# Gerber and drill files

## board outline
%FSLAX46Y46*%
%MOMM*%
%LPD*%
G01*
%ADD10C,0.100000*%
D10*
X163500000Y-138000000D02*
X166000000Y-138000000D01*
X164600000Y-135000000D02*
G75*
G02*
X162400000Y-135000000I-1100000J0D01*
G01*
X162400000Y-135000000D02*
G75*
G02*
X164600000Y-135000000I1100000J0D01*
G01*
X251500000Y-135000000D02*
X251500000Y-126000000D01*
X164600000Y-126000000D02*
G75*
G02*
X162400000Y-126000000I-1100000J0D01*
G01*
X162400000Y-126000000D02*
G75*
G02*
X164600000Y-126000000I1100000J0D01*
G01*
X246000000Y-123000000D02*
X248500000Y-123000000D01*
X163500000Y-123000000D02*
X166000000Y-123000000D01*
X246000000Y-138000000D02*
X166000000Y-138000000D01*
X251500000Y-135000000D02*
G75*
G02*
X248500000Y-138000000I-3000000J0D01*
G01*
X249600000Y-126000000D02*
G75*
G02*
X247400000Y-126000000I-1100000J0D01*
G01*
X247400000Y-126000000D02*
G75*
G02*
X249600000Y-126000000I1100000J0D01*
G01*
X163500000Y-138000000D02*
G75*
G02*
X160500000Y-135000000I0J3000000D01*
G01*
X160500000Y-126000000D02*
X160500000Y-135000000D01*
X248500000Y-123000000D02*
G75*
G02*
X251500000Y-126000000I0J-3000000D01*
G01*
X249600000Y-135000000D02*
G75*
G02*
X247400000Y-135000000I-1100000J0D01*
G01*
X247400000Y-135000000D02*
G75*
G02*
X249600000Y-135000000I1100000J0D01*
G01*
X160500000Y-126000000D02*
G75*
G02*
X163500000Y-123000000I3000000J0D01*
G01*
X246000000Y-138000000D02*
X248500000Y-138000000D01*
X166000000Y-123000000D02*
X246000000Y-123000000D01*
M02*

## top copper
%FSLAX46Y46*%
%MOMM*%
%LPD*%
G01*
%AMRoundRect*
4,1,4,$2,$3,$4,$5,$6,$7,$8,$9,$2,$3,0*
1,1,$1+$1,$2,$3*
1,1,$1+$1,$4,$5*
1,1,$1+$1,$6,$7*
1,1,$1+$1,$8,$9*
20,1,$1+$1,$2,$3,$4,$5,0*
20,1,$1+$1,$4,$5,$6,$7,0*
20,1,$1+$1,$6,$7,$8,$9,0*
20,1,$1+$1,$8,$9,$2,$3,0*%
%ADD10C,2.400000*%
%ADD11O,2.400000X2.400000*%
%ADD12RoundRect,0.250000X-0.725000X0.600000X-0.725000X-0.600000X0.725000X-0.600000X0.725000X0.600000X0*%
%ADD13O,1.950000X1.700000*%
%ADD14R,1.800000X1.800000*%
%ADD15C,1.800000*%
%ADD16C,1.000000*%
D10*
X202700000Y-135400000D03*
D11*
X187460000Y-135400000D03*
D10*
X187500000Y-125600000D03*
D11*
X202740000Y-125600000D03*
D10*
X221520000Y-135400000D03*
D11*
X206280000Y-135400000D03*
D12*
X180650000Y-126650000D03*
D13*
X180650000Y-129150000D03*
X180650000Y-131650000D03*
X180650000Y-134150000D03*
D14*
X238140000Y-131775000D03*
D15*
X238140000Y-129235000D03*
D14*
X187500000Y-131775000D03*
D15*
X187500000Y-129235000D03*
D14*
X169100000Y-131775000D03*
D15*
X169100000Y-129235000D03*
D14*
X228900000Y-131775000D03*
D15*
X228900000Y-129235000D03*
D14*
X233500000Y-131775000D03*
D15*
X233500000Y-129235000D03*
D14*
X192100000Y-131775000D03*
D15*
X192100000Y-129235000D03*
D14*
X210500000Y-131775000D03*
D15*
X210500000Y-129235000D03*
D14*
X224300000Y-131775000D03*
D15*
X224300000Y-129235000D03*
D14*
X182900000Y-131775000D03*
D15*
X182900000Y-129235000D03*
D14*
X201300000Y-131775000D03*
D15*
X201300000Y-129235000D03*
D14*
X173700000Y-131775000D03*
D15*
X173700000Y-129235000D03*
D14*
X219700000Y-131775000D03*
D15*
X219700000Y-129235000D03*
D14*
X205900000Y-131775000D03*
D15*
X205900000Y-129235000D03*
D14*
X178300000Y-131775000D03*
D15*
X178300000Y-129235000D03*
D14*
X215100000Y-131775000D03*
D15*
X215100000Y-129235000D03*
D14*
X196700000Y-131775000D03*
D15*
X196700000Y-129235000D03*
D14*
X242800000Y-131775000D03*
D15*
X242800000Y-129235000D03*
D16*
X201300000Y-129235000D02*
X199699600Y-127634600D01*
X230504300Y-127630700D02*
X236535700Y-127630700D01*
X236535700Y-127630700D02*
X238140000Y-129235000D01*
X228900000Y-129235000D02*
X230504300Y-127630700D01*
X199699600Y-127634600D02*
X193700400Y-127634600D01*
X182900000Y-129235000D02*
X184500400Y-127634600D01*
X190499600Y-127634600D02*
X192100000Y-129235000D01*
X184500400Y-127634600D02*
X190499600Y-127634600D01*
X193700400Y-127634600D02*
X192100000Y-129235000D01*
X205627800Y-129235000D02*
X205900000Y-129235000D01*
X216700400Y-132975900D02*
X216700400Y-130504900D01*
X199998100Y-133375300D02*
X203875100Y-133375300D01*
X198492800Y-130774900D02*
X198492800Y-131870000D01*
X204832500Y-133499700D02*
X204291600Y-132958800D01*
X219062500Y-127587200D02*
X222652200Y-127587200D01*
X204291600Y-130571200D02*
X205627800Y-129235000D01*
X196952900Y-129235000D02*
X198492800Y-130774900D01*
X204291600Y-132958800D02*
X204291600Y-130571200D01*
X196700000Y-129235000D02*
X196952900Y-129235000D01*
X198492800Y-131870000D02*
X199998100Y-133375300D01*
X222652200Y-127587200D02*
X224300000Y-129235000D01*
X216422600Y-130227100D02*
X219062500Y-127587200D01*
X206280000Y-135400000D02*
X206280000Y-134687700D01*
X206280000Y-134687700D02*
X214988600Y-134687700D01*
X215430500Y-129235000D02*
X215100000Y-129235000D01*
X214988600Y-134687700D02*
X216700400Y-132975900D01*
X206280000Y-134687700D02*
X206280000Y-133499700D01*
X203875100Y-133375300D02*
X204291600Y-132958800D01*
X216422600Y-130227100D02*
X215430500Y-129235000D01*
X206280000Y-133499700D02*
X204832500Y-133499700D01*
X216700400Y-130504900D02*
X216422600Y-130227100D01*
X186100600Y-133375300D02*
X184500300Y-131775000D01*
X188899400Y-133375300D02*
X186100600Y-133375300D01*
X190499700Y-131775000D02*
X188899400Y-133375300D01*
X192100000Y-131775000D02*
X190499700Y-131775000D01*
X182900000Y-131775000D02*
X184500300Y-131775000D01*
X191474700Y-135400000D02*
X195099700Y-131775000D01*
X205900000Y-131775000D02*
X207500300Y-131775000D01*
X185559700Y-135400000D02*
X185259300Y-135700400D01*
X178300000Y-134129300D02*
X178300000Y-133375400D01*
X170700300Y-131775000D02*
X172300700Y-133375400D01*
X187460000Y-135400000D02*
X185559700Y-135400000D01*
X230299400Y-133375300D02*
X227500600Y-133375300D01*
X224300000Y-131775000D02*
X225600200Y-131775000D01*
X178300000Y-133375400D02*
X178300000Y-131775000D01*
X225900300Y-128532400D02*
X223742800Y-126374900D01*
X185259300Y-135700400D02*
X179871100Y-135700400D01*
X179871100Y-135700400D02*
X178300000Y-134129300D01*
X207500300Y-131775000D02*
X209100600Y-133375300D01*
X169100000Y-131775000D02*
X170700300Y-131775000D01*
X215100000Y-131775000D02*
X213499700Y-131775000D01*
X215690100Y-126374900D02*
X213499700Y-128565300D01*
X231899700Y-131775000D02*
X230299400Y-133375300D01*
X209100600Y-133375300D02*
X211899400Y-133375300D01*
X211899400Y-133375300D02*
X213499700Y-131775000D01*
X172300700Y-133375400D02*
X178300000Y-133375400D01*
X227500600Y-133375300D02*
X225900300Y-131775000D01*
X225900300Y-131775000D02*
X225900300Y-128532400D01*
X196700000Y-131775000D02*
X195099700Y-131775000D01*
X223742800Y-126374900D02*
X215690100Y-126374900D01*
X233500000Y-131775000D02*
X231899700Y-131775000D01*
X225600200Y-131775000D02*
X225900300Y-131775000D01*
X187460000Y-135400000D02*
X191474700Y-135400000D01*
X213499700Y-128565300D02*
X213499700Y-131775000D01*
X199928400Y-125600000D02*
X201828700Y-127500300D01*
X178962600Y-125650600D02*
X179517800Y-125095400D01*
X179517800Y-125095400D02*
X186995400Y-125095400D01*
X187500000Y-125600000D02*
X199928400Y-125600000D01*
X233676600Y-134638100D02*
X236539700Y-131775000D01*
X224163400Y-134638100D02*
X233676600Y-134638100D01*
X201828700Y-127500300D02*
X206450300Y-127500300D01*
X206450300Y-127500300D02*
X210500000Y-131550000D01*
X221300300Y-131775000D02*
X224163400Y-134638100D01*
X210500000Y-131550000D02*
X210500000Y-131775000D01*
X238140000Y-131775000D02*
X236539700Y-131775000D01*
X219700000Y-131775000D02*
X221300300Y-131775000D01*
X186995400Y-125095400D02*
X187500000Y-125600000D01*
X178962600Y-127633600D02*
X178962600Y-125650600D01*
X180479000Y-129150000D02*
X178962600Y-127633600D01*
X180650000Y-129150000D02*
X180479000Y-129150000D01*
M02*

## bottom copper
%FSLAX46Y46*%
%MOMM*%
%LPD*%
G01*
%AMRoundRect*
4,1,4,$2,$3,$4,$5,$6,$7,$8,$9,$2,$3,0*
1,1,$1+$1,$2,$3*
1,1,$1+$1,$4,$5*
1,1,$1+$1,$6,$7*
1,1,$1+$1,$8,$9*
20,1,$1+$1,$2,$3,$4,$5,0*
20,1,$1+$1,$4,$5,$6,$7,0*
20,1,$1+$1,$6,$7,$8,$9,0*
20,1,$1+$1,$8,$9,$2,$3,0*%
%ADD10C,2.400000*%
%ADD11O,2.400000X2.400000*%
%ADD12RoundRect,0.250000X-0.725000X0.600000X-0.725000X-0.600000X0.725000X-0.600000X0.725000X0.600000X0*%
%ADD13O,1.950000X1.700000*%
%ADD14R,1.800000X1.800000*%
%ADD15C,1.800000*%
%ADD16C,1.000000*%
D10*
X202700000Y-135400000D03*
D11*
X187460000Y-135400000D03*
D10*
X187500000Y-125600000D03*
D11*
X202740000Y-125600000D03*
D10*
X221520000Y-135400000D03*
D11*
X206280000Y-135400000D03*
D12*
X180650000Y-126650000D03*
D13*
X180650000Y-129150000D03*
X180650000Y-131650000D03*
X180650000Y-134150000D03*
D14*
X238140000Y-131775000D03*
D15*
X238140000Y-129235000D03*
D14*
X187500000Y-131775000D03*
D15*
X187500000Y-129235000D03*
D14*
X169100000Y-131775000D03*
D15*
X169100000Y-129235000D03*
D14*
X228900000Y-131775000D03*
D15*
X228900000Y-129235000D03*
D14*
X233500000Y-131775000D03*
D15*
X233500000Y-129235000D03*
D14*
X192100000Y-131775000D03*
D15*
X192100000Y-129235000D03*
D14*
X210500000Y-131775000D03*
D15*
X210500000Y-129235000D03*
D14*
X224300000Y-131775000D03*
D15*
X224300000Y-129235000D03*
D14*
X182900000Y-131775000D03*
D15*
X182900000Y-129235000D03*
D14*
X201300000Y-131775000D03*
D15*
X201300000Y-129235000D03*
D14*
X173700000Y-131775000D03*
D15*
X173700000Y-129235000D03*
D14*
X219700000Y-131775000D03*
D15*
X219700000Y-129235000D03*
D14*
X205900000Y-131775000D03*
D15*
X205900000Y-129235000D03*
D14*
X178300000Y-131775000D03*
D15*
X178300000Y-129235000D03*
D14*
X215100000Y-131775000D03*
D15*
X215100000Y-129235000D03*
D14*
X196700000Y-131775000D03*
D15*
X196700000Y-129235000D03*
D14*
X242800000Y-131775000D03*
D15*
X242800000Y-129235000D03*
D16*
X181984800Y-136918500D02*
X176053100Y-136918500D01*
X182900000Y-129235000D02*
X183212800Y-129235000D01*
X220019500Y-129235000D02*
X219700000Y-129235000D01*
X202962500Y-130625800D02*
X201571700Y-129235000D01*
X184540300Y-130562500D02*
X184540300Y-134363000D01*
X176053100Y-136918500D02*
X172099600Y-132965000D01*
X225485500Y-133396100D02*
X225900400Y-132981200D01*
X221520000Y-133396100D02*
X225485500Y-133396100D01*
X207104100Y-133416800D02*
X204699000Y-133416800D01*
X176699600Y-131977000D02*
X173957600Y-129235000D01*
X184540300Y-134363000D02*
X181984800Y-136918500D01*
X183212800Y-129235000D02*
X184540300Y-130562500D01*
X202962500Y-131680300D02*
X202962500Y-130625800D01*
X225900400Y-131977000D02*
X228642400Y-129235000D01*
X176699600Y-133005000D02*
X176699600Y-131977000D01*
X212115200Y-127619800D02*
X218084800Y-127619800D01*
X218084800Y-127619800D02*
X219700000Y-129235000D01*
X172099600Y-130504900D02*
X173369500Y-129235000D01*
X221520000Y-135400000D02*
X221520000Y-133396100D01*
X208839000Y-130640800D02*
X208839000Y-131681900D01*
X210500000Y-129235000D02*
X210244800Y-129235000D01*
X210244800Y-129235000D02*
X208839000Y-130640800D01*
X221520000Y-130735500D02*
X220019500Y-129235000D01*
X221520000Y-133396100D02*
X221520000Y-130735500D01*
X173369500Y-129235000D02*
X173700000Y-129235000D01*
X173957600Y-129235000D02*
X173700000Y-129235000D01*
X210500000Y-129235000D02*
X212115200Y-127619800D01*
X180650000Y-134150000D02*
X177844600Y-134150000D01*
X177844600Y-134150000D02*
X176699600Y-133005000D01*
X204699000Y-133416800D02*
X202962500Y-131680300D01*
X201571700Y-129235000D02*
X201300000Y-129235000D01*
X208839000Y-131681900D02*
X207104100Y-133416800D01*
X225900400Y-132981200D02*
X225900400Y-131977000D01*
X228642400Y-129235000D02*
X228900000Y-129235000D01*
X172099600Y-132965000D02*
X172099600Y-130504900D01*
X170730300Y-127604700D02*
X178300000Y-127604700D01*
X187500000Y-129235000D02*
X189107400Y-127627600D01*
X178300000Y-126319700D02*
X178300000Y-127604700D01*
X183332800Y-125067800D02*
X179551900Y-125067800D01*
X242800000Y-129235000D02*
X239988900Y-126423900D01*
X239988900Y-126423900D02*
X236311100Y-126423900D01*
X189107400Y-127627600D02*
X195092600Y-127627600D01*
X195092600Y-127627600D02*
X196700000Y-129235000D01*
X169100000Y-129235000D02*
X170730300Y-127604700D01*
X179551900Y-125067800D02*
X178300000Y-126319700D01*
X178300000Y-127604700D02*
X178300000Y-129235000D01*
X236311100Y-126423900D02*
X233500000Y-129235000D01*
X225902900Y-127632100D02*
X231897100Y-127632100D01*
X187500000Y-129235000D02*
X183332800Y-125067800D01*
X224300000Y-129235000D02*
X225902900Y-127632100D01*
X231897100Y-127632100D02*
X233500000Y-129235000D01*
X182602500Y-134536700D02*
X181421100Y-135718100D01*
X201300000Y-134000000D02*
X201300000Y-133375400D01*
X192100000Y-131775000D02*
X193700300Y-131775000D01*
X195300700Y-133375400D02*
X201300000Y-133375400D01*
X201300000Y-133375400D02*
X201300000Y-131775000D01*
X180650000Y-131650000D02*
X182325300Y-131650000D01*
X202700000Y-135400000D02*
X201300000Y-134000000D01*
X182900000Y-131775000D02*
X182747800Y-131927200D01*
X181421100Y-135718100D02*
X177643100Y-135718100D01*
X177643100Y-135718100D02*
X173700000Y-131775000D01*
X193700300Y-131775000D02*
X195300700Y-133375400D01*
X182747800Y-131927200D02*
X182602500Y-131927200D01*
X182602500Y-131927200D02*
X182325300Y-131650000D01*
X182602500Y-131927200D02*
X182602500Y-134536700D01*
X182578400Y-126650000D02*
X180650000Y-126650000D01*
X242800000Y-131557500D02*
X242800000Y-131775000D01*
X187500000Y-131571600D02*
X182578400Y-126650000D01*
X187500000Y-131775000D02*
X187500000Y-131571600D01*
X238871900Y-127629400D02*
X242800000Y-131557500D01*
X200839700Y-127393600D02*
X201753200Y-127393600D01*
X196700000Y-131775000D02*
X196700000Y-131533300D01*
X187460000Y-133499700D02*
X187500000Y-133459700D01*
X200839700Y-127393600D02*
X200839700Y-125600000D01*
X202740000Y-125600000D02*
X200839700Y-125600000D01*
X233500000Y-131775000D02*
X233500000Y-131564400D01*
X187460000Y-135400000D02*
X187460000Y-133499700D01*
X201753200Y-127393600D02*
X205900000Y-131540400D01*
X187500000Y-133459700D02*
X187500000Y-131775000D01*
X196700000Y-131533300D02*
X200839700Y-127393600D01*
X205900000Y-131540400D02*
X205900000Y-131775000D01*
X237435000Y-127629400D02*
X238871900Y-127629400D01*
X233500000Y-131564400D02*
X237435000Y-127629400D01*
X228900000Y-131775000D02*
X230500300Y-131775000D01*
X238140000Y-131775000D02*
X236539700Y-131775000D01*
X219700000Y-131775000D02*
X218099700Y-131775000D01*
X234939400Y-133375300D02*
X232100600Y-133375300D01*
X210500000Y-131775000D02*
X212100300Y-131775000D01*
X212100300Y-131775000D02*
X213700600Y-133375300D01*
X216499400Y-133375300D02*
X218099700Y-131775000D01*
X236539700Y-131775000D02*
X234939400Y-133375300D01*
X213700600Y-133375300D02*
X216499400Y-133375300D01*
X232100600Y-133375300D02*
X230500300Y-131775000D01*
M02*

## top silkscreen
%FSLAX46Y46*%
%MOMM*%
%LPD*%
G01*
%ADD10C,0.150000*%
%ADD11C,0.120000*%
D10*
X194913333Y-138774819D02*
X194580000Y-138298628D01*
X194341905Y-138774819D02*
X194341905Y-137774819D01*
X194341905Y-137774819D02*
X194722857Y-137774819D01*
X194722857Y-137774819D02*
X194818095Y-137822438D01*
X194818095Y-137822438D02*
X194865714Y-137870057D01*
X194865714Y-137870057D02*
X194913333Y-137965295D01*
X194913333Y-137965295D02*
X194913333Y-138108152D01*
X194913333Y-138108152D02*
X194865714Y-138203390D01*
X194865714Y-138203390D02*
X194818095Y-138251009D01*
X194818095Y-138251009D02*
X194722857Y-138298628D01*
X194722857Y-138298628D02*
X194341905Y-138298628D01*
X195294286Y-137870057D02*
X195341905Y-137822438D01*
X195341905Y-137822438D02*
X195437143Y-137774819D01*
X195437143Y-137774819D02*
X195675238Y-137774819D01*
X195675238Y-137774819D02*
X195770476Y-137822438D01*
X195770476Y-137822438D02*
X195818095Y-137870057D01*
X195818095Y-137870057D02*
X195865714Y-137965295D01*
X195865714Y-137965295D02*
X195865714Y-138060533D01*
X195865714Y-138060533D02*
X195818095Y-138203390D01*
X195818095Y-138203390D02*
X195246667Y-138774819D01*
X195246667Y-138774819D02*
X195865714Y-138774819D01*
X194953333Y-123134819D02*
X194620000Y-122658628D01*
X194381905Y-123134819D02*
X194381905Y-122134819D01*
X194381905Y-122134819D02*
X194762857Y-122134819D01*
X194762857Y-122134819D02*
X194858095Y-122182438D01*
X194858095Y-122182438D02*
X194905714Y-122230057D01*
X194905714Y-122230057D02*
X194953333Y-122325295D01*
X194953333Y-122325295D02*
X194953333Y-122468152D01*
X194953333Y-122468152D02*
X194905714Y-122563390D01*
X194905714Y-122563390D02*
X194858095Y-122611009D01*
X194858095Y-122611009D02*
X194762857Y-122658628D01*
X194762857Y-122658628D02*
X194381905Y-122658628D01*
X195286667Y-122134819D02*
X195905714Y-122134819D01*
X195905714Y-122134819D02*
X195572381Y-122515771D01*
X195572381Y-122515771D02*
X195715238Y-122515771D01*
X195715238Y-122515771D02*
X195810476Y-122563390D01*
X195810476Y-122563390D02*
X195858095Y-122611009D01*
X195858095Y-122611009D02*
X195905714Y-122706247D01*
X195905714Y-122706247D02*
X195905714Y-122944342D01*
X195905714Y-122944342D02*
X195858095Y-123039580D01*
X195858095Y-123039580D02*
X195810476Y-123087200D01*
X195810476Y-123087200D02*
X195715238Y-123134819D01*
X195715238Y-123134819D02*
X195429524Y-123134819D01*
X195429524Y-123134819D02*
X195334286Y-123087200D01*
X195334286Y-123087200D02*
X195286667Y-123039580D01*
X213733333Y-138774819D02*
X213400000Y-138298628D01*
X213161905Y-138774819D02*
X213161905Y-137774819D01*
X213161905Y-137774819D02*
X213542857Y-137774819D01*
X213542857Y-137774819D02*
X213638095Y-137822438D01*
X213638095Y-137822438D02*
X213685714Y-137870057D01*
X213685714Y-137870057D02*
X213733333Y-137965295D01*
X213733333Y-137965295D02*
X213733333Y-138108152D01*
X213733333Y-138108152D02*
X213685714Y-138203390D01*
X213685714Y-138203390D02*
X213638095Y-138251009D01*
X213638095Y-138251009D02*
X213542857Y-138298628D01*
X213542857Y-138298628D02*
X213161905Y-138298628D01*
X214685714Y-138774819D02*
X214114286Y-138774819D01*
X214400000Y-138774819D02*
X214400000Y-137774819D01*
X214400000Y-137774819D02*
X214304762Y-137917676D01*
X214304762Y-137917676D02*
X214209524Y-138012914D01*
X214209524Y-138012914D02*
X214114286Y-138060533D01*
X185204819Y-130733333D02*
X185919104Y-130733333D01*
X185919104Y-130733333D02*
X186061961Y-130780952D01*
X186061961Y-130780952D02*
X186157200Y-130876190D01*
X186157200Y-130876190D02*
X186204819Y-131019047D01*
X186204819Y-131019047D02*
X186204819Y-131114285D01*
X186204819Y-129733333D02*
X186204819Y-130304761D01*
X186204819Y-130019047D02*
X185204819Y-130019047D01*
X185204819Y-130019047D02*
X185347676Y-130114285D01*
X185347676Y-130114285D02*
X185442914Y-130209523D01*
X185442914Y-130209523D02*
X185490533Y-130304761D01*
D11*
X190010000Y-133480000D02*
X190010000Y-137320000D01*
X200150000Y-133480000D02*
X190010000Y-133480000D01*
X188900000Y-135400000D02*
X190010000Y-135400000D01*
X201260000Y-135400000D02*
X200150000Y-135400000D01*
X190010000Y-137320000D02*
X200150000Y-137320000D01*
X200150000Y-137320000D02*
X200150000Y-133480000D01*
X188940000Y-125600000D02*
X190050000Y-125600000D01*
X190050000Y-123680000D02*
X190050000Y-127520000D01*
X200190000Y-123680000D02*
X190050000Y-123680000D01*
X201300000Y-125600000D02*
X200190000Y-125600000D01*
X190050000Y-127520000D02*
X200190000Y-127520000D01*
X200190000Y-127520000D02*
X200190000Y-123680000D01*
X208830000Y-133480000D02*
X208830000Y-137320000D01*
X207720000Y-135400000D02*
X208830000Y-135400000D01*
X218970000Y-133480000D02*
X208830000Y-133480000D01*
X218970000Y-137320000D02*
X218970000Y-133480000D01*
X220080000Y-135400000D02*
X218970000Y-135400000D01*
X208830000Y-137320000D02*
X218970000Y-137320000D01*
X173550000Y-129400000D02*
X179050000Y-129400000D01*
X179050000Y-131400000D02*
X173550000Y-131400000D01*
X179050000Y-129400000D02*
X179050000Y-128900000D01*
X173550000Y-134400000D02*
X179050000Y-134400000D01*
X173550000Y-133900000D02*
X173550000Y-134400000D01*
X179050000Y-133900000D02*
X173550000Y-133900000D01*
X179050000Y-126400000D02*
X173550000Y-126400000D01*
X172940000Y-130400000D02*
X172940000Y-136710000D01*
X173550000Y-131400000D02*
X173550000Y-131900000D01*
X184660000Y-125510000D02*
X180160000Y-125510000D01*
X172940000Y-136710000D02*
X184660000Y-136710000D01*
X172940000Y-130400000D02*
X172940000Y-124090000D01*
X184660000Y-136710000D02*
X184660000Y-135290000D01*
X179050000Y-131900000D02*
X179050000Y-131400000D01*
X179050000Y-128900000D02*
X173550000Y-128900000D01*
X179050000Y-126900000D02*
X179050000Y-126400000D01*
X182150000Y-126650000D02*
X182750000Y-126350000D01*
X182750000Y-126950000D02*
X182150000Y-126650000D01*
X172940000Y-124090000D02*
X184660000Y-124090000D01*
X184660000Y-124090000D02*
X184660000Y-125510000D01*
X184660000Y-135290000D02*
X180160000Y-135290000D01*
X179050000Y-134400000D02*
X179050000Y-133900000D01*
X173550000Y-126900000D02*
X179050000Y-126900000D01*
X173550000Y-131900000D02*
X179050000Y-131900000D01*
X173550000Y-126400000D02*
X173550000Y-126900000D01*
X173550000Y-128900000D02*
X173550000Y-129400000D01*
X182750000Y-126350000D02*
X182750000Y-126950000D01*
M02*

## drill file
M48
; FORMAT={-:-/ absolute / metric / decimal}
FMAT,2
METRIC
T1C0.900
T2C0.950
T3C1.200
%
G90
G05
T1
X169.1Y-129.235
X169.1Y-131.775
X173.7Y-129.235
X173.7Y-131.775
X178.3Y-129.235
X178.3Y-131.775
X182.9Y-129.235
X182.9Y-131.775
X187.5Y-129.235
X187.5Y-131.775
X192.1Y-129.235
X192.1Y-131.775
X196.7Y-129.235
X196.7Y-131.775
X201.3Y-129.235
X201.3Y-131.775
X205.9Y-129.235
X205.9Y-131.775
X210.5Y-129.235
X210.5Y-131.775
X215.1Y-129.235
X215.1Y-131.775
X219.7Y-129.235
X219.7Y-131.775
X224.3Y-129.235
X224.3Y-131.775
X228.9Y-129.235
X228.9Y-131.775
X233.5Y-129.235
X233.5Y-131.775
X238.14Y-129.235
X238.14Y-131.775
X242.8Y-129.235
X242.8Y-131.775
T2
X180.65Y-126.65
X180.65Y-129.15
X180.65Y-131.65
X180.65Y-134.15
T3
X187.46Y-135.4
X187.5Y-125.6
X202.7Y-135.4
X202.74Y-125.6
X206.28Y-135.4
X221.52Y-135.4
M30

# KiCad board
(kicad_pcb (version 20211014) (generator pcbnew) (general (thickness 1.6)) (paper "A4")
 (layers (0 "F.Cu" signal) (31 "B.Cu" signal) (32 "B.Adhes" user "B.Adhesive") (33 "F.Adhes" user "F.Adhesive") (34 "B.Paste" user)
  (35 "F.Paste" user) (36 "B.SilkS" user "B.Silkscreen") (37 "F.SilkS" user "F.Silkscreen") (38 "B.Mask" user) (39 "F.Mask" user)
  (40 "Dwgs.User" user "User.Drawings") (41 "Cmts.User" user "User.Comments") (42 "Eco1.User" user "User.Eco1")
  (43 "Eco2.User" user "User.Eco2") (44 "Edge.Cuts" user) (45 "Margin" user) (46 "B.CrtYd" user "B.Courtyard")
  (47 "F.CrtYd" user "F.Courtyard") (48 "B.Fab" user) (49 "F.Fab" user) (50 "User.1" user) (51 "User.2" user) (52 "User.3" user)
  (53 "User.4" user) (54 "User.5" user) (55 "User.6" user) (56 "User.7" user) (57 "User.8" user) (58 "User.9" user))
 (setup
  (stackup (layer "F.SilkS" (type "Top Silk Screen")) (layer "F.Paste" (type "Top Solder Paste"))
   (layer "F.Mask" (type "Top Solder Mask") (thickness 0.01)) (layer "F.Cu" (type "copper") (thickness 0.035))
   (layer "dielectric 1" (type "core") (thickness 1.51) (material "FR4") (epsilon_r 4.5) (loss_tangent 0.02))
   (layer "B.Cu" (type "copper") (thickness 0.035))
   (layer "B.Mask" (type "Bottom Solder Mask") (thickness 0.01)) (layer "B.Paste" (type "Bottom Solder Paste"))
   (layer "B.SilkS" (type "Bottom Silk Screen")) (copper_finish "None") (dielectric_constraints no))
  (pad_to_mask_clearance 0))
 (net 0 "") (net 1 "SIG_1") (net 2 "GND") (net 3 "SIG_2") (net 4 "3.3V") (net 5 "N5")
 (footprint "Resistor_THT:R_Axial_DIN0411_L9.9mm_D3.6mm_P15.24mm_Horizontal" (layer "F.Cu") (at 202.7 135.4 180)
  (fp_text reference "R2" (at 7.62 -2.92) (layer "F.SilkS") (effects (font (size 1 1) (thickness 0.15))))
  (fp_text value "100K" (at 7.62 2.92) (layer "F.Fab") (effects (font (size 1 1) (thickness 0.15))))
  (fp_line (start 12.69 1.92) (end 12.69 -1.92) (layer "F.SilkS") (width 0.12))
  (fp_line (start 2.55 1.92) (end 12.69 1.92) (layer "F.SilkS") (width 0.12))
  (fp_line (start 13.8 0) (end 12.69 0) (layer "F.SilkS") (width 0.12))
  (fp_line (start 1.44 0) (end 2.55 0) (layer "F.SilkS") (width 0.12))
  (fp_line (start 12.69 -1.92) (end 2.55 -1.92) (layer "F.SilkS") (width 0.12))
  (fp_line (start 2.55 -1.92) (end 2.55 1.92) (layer "F.SilkS") (width 0.12))
  (pad "1" thru_hole circle (at 0 0 180) (size 2.4 2.4) (drill 1.2) (layers *.Cu *.Mask) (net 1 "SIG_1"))
  (pad "2" thru_hole oval (at 15.24 0 180) (size 2.4 2.4) (drill 1.2) (layers *.Cu *.Mask) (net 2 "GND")))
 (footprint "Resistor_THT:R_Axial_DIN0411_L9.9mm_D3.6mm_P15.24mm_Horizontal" (layer "F.Cu") (at 187.5 125.6)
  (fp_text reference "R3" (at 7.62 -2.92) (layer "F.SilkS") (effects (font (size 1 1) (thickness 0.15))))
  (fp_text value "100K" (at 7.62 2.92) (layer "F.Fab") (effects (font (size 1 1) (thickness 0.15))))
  (fp_line (start 1.44 0) (end 2.55 0) (layer "F.SilkS") (width 0.12))
  (fp_line (start 2.55 -1.92) (end 2.55 1.92) (layer "F.SilkS") (width 0.12))
  (fp_line (start 12.69 -1.92) (end 2.55 -1.92) (layer "F.SilkS") (width 0.12))
  (fp_line (start 13.8 0) (end 12.69 0) (layer "F.SilkS") (width 0.12))
  (fp_line (start 2.55 1.92) (end 12.69 1.92) (layer "F.SilkS") (width 0.12))
  (fp_line (start 12.69 1.92) (end 12.69 -1.92) (layer "F.SilkS") (width 0.12))
  (pad "1" thru_hole circle (at 0 0) (size 2.4 2.4) (drill 1.2) (layers *.Cu *.Mask) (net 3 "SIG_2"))
  (pad "2" thru_hole oval (at 15.24 0) (size 2.4 2.4) (drill 1.2) (layers *.Cu *.Mask) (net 2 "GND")))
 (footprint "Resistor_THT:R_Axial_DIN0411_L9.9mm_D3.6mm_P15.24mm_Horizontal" (layer "F.Cu") (at 221.52 135.4 180)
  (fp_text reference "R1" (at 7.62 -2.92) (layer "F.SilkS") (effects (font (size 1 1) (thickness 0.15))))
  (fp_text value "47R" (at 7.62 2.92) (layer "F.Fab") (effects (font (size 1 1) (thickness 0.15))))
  (fp_line (start 12.69 1.92) (end 12.69 -1.92) (layer "F.SilkS") (width 0.12))
  (fp_line (start 13.8 0) (end 12.69 0) (layer "F.SilkS") (width 0.12))
  (fp_line (start 2.55 1.92) (end 12.69 1.92) (layer "F.SilkS") (width 0.12))
  (fp_line (start 2.55 -1.92) (end 2.55 1.92) (layer "F.SilkS") (width 0.12))
  (fp_line (start 1.44 0) (end 2.55 0) (layer "F.SilkS") (width 0.12))
  (fp_line (start 12.69 -1.92) (end 2.55 -1.92) (layer "F.SilkS") (width 0.12))
  (pad "1" thru_hole circle (at 0 0 180) (size 2.4 2.4) (drill 1.2) (layers *.Cu *.Mask) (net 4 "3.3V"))
  (pad "2" thru_hole oval (at 15.24 0 180) (size 2.4 2.4) (drill 1.2) (layers *.Cu *.Mask) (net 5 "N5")))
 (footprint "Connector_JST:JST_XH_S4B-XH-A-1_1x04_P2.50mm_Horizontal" (layer "F.Cu") (at 180.65 126.65 -90)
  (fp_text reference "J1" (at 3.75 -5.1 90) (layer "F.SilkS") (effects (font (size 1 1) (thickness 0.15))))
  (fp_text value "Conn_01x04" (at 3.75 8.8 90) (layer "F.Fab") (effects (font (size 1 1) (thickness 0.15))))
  (fp_line (start 2.75 7.1) (end 2.75 1.6) (layer "F.SilkS") (width 0.12))
  (fp_line (start 4.75 1.6) (end 4.75 7.1) (layer "F.SilkS") (width 0.12))
  (fp_line (start 2.75 1.6) (end 2.25 1.6) (layer "F.SilkS") (width 0.12))
  (fp_line (start 7.75 7.1) (end 7.75 1.6) (layer "F.SilkS") (width 0.12))
  (fp_line (start 7.25 7.1) (end 7.75 7.1) (layer "F.SilkS") (width 0.12))
  (fp_line (start 7.25 1.6) (end 7.25 7.1) (layer "F.SilkS") (width 0.12))
  (fp_line (start -0.25 1.6) (end -0.25 7.1) (layer "F.SilkS") (width 0.12))
  (fp_line (start 3.75 7.71) (end 10.06 7.71) (layer "F.SilkS") (width 0.12))
  (fp_line (start 4.75 7.1) (end 5.25 7.1) (layer "F.SilkS") (width 0.12))
  (fp_line (start -1.14 -4.01) (end -1.14 0.49) (layer "F.SilkS") (width 0.12))
  (fp_line (start 10.06 7.71) (end 10.06 -4.01) (layer "F.SilkS") (width 0.12))
  (fp_line (start 3.75 7.71) (end -2.56 7.71) (layer "F.SilkS") (width 0.12))
  (fp_line (start 10.06 -4.01) (end 8.64 -4.01) (layer "F.SilkS") (width 0.12))
  (fp_line (start 5.25 1.6) (end 4.75 1.6) (layer "F.SilkS") (width 0.12))
  (fp_line (start 2.25 1.6) (end 2.25 7.1) (layer "F.SilkS") (width 0.12))
  (fp_line (start 0.25 1.6) (end -0.25 1.6) (layer "F.SilkS") (width 0.12))
  (fp_line (start 0 -1.5) (end -0.3 -2.1) (layer "F.SilkS") (width 0.12))
  (fp_line (start 0.3 -2.1) (end 0 -1.5) (layer "F.SilkS") (width 0.12))
  (fp_line (start -2.56 7.71) (end -2.56 -4.01) (layer "F.SilkS") (width 0.12))
  (fp_line (start -2.56 -4.01) (end -1.14 -4.01) (layer "F.SilkS") (width 0.12))
  (fp_line (start 8.64 -4.01) (end 8.64 0.49) (layer "F.SilkS") (width 0.12))
  (fp_line (start 7.75 1.6) (end 7.25 1.6) (layer "F.SilkS") (width 0.12))
  (fp_line (start 0.25 7.1) (end 0.25 1.6) (layer "F.SilkS") (width 0.12))
  (fp_line (start 5.25 7.1) (end 5.25 1.6) (layer "F.SilkS") (width 0.12))
  (fp_line (start -0.25 7.1) (end 0.25 7.1) (layer "F.SilkS") (width 0.12))
  (fp_line (start 2.25 7.1) (end 2.75 7.1) (layer "F.SilkS") (width 0.12))
  (fp_line (start -0.3 -2.1) (end 0.3 -2.1) (layer "F.SilkS") (width 0.12))
  (pad "1" thru_hole roundrect (at 0 0 270) (size 1.7 1.95) (drill 0.95) (layers *.Cu *.Mask) (roundrect_rratio 0.1470588235) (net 2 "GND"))
  (pad "2" thru_hole oval (at 2.5 0 270) (size 1.7 1.95) (drill 0.95) (layers *.Cu *.Mask) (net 3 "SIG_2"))
  (pad "3" thru_hole oval (at 5 0 270) (size 1.7 1.95) (drill 0.95) (layers *.Cu *.Mask) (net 1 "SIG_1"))
  (pad "4" thru_hole oval (at 7.5 0 270) (size 1.7 1.95) (drill 0.95) (layers *.Cu *.Mask) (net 4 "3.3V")))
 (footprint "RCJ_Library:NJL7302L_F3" (layer "B.Cu") (at 238.14 131.775 90)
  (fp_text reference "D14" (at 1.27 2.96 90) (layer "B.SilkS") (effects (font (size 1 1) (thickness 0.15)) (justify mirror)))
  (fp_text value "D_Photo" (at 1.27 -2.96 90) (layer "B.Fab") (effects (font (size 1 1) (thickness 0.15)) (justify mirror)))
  (pad "1" thru_hole rect (at 0 0 90) (size 1.8 1.8) (drill 0.9) (layers *.Cu *.Mask) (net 3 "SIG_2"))
  (pad "2" thru_hole circle (at 2.54 0 90) (size 1.8 1.8) (drill 0.9) (layers *.Cu *.Mask) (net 4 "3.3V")))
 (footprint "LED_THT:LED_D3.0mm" (layer "B.Cu") (at 187.5 131.775 90)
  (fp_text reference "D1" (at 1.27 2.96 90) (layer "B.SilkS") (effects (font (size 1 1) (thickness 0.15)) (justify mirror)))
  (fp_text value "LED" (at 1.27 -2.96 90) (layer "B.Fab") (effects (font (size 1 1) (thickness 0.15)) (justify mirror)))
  (pad "1" thru_hole rect (at 0 0 90) (size 1.8 1.8) (drill 0.9) (layers *.Cu *.Mask) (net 2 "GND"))
  (pad "2" thru_hole circle (at 2.54 0 90) (size 1.8 1.8) (drill 0.9) (layers *.Cu *.Mask) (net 5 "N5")))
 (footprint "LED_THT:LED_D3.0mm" (layer "B.Cu") (at 169.1 131.775 90)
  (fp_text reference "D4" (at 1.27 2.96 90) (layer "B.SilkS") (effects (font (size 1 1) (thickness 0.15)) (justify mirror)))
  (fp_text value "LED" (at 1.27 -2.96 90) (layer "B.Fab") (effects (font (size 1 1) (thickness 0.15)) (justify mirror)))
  (pad "1" thru_hole rect (at 0 0 90) (size 1.8 1.8) (drill 0.9) (layers *.Cu *.Mask) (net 2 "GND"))
  (pad "2" thru_hole circle (at 2.54 0 90) (size 1.8 1.8) (drill 0.9) (layers *.Cu *.Mask) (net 5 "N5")))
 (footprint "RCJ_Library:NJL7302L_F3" (layer "B.Cu") (at 228.9 131.775 90)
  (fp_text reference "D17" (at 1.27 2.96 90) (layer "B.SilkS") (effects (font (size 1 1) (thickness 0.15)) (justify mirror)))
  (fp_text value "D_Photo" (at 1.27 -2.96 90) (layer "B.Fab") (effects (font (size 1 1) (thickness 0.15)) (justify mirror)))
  (pad "1" thru_hole rect (at 0 0 90) (size 1.8 1.8) (drill 0.9) (layers *.Cu *.Mask) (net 3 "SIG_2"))
  (pad "2" thru_hole circle (at 2.54 0 90) (size 1.8 1.8) (drill 0.9) (layers *.Cu *.Mask) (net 4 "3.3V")))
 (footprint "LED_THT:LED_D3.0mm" (layer "B.Cu") (at 233.5 131.775 90)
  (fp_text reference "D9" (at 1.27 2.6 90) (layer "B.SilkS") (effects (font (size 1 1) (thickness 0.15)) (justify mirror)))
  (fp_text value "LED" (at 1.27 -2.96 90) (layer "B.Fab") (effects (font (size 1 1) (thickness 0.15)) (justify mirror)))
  (pad "1" thru_hole rect (at 0 0 90) (size 1.8 1.8) (drill 0.9) (layers *.Cu *.Mask) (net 2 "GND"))
  (pad "2" thru_hole circle (at 2.54 0 90) (size 1.8 1.8) (drill 0.9) (layers *.Cu *.Mask) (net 5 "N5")))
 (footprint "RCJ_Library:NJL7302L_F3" (layer "B.Cu") (at 192.1 131.775 90)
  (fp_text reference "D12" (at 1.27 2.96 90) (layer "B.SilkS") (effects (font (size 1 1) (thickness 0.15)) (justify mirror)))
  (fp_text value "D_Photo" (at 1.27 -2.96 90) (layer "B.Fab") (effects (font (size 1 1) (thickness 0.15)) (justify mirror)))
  (pad "1" thru_hole rect (at 0 0 90) (size 1.8 1.8) (drill 0.9) (layers *.Cu *.Mask) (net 1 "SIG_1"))
  (pad "2" thru_hole circle (at 2.54 0 90) (size 1.8 1.8) (drill 0.9) (layers *.Cu *.Mask) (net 4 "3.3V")))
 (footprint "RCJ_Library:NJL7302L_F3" (layer "B.Cu") (at 210.5 131.775 90)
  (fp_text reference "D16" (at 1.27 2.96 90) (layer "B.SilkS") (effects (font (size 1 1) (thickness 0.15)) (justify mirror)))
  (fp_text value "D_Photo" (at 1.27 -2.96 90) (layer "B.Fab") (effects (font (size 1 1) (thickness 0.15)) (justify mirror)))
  (pad "1" thru_hole rect (at 0 0 90) (size 1.8 1.8) (drill 0.9) (layers *.Cu *.Mask) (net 3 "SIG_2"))
  (pad "2" thru_hole circle (at 2.54 0 90) (size 1.8 1.8) (drill 0.9) (layers *.Cu *.Mask) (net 4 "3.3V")))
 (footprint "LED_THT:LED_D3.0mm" (layer "B.Cu") (at 224.3 131.775 90)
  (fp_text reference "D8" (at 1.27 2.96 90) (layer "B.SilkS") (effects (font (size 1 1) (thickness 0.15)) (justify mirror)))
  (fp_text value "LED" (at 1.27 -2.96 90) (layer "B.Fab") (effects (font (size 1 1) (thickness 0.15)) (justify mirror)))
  (pad "1" thru_hole rect (at 0 0 90) (size 1.8 1.8) (drill 0.9) (layers *.Cu *.Mask) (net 2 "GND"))
  (pad "2" thru_hole circle (at 2.54 0 90) (size 1.8 1.8) (drill 0.9) (layers *.Cu *.Mask) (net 5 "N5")))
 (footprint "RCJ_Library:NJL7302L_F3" (layer "B.Cu") (at 182.9 131.775 90)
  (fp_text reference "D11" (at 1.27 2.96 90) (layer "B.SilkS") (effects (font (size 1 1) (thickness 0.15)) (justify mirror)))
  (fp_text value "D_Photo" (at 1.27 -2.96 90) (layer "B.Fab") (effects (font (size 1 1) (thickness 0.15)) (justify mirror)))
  (pad "1" thru_hole rect (at 0 0 90) (size 1.8 1.8) (drill 0.9) (layers *.Cu *.Mask) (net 1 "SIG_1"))
  (pad "2" thru_hole circle (at 2.54 0 90) (size 1.8 1.8) (drill 0.9) (layers *.Cu *.Mask) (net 4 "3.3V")))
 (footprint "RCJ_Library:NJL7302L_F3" (layer "B.Cu") (at 201.3 131.775 90)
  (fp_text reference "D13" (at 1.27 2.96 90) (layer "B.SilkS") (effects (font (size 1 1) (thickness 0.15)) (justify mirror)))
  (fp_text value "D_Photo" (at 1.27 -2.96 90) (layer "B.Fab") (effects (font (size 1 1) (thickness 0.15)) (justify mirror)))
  (pad "1" thru_hole rect (at 0 0 90) (size 1.8 1.8) (drill 0.9) (layers *.Cu *.Mask) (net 1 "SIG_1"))
  (pad "2" thru_hole circle (at 2.54 0 90) (size 1.8 1.8) (drill 0.9) (layers *.Cu *.Mask) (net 4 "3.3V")))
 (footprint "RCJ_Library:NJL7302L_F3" (layer "B.Cu") (at 173.7 131.775 90)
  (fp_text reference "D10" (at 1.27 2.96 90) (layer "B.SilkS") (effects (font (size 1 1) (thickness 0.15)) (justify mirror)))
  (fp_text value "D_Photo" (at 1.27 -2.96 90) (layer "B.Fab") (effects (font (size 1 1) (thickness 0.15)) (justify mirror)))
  (pad "1" thru_hole rect (at 0 0 90) (size 1.8 1.8) (drill 0.9) (layers *.Cu *.Mask) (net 1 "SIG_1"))
  (pad "2" thru_hole circle (at 2.54 0 90) (size 1.8 1.8) (drill 0.9) (layers *.Cu *.Mask) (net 4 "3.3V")))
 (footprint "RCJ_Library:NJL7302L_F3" (layer "B.Cu") (at 219.7 131.775 90)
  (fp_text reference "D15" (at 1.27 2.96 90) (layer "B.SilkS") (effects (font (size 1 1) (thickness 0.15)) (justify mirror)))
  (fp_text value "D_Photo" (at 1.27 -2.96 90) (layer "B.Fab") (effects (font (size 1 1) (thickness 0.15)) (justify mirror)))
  (pad "1" thru_hole rect (at 0 0 90) (size 1.8 1.8) (drill 0.9) (layers *.Cu *.Mask) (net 3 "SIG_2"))
  (pad "2" thru_hole circle (at 2.54 0 90) (size 1.8 1.8) (drill 0.9) (layers *.Cu *.Mask) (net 4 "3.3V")))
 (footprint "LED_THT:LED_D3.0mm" (layer "B.Cu") (at 205.9 131.775 90)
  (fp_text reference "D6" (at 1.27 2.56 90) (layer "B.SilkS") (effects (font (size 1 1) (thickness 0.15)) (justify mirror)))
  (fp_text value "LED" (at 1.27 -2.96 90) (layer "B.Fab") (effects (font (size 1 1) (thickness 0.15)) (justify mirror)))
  (pad "1" thru_hole rect (at 0 0 90) (size 1.8 1.8) (drill 0.9) (layers *.Cu *.Mask) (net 2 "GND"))
  (pad "2" thru_hole circle (at 2.54 0 90) (size 1.8 1.8) (drill 0.9) (layers *.Cu *.Mask) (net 5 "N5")))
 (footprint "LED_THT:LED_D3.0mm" (layer "B.Cu") (at 178.3 131.775 90)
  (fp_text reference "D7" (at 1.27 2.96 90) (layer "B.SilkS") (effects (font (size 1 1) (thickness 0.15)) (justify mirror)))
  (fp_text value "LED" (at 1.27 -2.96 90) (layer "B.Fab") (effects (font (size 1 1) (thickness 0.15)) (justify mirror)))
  (pad "1" thru_hole rect (at 0 0 90) (size 1.8 1.8) (drill 0.9) (layers *.Cu *.Mask) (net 2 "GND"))
  (pad "2" thru_hole circle (at 2.54 0 90) (size 1.8 1.8) (drill 0.9) (layers *.Cu *.Mask) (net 5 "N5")))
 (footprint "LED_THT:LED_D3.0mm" (layer "B.Cu") (at 215.1 131.775 90)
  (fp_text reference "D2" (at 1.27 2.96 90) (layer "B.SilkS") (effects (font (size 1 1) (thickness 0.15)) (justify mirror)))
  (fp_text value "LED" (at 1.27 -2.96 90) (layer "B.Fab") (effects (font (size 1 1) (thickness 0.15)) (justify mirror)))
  (pad "1" thru_hole rect (at 0 0 90) (size 1.8 1.8) (drill 0.9) (layers *.Cu *.Mask) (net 2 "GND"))
  (pad "2" thru_hole circle (at 2.54 0 90) (size 1.8 1.8) (drill 0.9) (layers *.Cu *.Mask) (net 5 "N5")))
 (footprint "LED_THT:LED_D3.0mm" (layer "B.Cu") (at 196.7 131.775 90)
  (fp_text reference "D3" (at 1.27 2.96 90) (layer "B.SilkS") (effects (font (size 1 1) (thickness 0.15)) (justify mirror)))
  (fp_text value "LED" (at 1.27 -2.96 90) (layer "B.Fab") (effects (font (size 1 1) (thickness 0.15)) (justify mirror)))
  (pad "1" thru_hole rect (at 0 0 90) (size 1.8 1.8) (drill 0.9) (layers *.Cu *.Mask) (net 2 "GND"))
  (pad "2" thru_hole circle (at 2.54 0 90) (size 1.8 1.8) (drill 0.9) (layers *.Cu *.Mask) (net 5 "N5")))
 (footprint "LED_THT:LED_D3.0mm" (layer "B.Cu") (at 242.8 131.775 90)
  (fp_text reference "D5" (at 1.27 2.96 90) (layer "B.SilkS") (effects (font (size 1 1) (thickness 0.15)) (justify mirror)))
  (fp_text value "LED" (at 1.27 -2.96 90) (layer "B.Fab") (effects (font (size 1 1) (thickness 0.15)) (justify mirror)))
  (pad "1" thru_hole rect (at 0 0 90) (size 1.8 1.8) (drill 0.9) (layers *.Cu *.Mask) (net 2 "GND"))
  (pad "2" thru_hole circle (at 2.54 0 90) (size 1.8 1.8) (drill 0.9) (layers *.Cu *.Mask) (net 5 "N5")))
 (gr_line (start 163.5 138) (end 166 138) (layer "Edge.Cuts") (width 0.1))
 (gr_circle (center 163.5 135) (end 162.4 135) (layer "Edge.Cuts") (width 0.1) (fill none))
 (gr_line (start 251.5 135) (end 251.5 126) (layer "Edge.Cuts") (width 0.1))
 (gr_circle (center 163.5 126) (end 162.4 126) (layer "Edge.Cuts") (width 0.1) (fill none))
 (gr_line (start 246 123) (end 248.5 123) (layer "Edge.Cuts") (width 0.1))
 (gr_line (start 163.5 123) (end 166 123) (layer "Edge.Cuts") (width 0.1))
 (gr_line (start 246 138) (end 166 138) (layer "Edge.Cuts") (width 0.1))
 (gr_arc (start 251.5 135) (mid 250.62132 137.12132) (end 248.5 138) (layer "Edge.Cuts") (width 0.1))
 (gr_circle (center 248.5 126) (end 249.6 126) (layer "Edge.Cuts") (width 0.1) (fill none))
 (gr_arc (start 163.5 138) (mid 161.37868 137.12132) (end 160.5 135) (layer "Edge.Cuts") (width 0.1))
 (gr_line (start 160.5 126) (end 160.5 135) (layer "Edge.Cuts") (width 0.1))
 (gr_arc (start 248.5 123) (mid 250.62132 123.87868) (end 251.5 126) (layer "Edge.Cuts") (width 0.1))
 (gr_circle (center 248.5 135) (end 249.6 135) (layer "Edge.Cuts") (width 0.1) (fill none))
 (gr_arc (start 160.5 126) (mid 161.37868 123.87868) (end 163.5 123) (layer "Edge.Cuts") (width 0.1))
 (gr_line (start 246 138) (end 248.5 138) (layer "Edge.Cuts") (width 0.1))
 (gr_line (start 166 123) (end 246 123) (layer "Edge.Cuts") (width 0.1))
 (segment (start 201.3 129.235) (end 199.6996 127.6346) (width 1) (layer "F.Cu") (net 4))
 (segment (start 230.5043 127.6307) (end 236.5357 127.6307) (width 1) (layer "F.Cu") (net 4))
 (segment (start 236.5357 127.6307) (end 238.14 129.235) (width 1) (layer "F.Cu") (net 4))
 (segment (start 228.9 129.235) (end 230.5043 127.6307) (width 1) (layer "F.Cu") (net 4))
 (segment (start 199.6996 127.6346) (end 193.7004 127.6346) (width 1) (layer "F.Cu") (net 4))
 (segment (start 182.9 129.235) (end 184.5004 127.6346) (width 1) (layer "F.Cu") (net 4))
 (segment (start 190.4996 127.6346) (end 192.1 129.235) (width 1) (layer "F.Cu") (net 4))
 (segment (start 184.5004 127.6346) (end 190.4996 127.6346) (width 1) (layer "F.Cu") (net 4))
 (segment (start 193.7004 127.6346) (end 192.1 129.235) (width 1) (layer "F.Cu") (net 4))
 (segment (start 181.9848 136.9185) (end 176.0531 136.9185) (width 1) (layer "B.Cu") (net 4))
 (segment (start 182.9 129.235) (end 183.2128 129.235) (width 1) (layer "B.Cu") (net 4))
 (segment (start 220.0195 129.235) (end 219.7 129.235) (width 1) (layer "B.Cu") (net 4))
 (segment (start 202.9625 130.6258) (end 201.5717 129.235) (width 1) (layer "B.Cu") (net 4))
 (segment (start 184.5403 130.5625) (end 184.5403 134.363) (width 1) (layer "B.Cu") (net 4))
 (segment (start 176.0531 136.9185) (end 172.0996 132.965) (width 1) (layer "B.Cu") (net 4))
 (segment (start 225.4855 133.3961) (end 225.9004 132.9812) (width 1) (layer "B.Cu") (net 4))
 (segment (start 221.52 133.3961) (end 225.4855 133.3961) (width 1) (layer "B.Cu") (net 4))
 (segment (start 207.1041 133.4168) (end 204.699 133.4168) (width 1) (layer "B.Cu") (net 4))
 (segment (start 176.6996 131.977) (end 173.9576 129.235) (width 1) (layer "B.Cu") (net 4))
 (segment (start 184.5403 134.363) (end 181.9848 136.9185) (width 1) (layer "B.Cu") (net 4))
 (segment (start 183.2128 129.235) (end 184.5403 130.5625) (width 1) (layer "B.Cu") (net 4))
 (segment (start 202.9625 131.6803) (end 202.9625 130.6258) (width 1) (layer "B.Cu") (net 4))
 (segment (start 225.9004 131.977) (end 228.6424 129.235) (width 1) (layer "B.Cu") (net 4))
 (segment (start 176.6996 133.005) (end 176.6996 131.977) (width 1) (layer "B.Cu") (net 4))
 (segment (start 212.1152 127.6198) (end 218.0848 127.6198) (width 1) (layer "B.Cu") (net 4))
 (segment (start 218.0848 127.6198) (end 219.7 129.235) (width 1) (layer "B.Cu") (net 4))
 (segment (start 172.0996 130.5049) (end 173.3695 129.235) (width 1) (layer "B.Cu") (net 4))
 (segment (start 221.52 135.4) (end 221.52 133.3961) (width 1) (layer "B.Cu") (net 4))
 (segment (start 208.839 130.6408) (end 208.839 131.6819) (width 1) (layer "B.Cu") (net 4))
 (segment (start 210.5 129.235) (end 210.2448 129.235) (width 1) (layer "B.Cu") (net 4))
 (segment (start 210.2448 129.235) (end 208.839 130.6408) (width 1) (layer "B.Cu") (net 4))
 (segment (start 221.52 130.7355) (end 220.0195 129.235) (width 1) (layer "B.Cu") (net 4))
 (segment (start 221.52 133.3961) (end 221.52 130.7355) (width 1) (layer "B.Cu") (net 4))
 (segment (start 173.3695 129.235) (end 173.7 129.235) (width 1) (layer "B.Cu") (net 4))
 (segment (start 173.9576 129.235) (end 173.7 129.235) (width 1) (layer "B.Cu") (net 4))
 (segment (start 210.5 129.235) (end 212.1152 127.6198) (width 1) (layer "B.Cu") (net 4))
 (segment (start 180.65 134.15) (end 177.8446 134.15) (width 1) (layer "B.Cu") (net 4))
 (segment (start 177.8446 134.15) (end 176.6996 133.005) (width 1) (layer "B.Cu") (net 4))
 (segment (start 204.699 133.4168) (end 202.9625 131.6803) (width 1) (layer "B.Cu") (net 4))
 (segment (start 201.5717 129.235) (end 201.3 129.235) (width 1) (layer "B.Cu") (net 4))
 (segment (start 208.839 131.6819) (end 207.1041 133.4168) (width 1) (layer "B.Cu") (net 4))
 (segment (start 225.9004 132.9812) (end 225.9004 131.977) (width 1) (layer "B.Cu") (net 4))
 (segment (start 228.6424 129.235) (end 228.9 129.235) (width 1) (layer "B.Cu") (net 4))
 (segment (start 172.0996 132.965) (end 172.0996 130.5049) (width 1) (layer "B.Cu") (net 4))
 (segment (start 205.6278 129.235) (end 205.9 129.235) (width 1) (layer "F.Cu") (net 5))
 (segment (start 216.7004 132.9759) (end 216.7004 130.5049) (width 1) (layer "F.Cu") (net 5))
 (segment (start 199.9981 133.3753) (end 203.8751 133.3753) (width 1) (layer "F.Cu") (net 5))
 (segment (start 198.4928 130.7749) (end 198.4928 131.87) (width 1) (layer "F.Cu") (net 5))
 (segment (start 204.8325 133.4997) (end 204.2916 132.9588) (width 1) (layer "F.Cu") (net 5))
 (segment (start 219.0625 127.5872) (end 222.6522 127.5872) (width 1) (layer "F.Cu") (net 5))
 (segment (start 204.2916 130.5712) (end 205.6278 129.235) (width 1) (layer "F.Cu") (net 5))
 (segment (start 196.9529 129.235) (end 198.4928 130.7749) (width 1) (layer "F.Cu") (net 5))
 (segment (start 204.2916 132.9588) (end 204.2916 130.5712) (width 1) (layer "F.Cu") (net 5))
 (segment (start 196.7 129.235) (end 196.9529 129.235) (width 1) (layer "F.Cu") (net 5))
 (segment (start 198.4928 131.87) (end 199.9981 133.3753) (width 1) (layer "F.Cu") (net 5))
 (segment (start 222.6522 127.5872) (end 224.3 129.235) (width 1) (layer "F.Cu") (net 5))
 (segment (start 216.4226 130.2271) (end 219.0625 127.5872) (width 1) (layer "F.Cu") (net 5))
 (segment (start 206.28 135.4) (end 206.28 134.6877) (width 1) (layer "F.Cu") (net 5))
 (segment (start 206.28 134.6877) (end 214.9886 134.6877) (width 1) (layer "F.Cu") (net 5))
 (segment (start 215.4305 129.235) (end 215.1 129.235) (width 1) (layer "F.Cu") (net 5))
 (segment (start 214.9886 134.6877) (end 216.7004 132.9759) (width 1) (layer "F.Cu") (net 5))
 (segment (start 206.28 134.6877) (end 206.28 133.4997) (width 1) (layer "F.Cu") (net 5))
 (segment (start 203.8751 133.3753) (end 204.2916 132.9588) (width 1) (layer "F.Cu") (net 5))
 (segment (start 216.4226 130.2271) (end 215.4305 129.235) (width 1) (layer "F.Cu") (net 5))
 (segment (start 206.28 133.4997) (end 204.8325 133.4997) (width 1) (layer "F.Cu") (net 5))
 (segment (start 216.7004 130.5049) (end 216.4226 130.2271) (width 1) (layer "F.Cu") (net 5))
 (segment (start 170.7303 127.6047) (end 178.3 127.6047) (width 1) (layer "B.Cu") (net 5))
 (segment (start 187.5 129.235) (end 189.1074 127.6276) (width 1) (layer "B.Cu") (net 5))
 (segment (start 178.3 126.3197) (end 178.3 127.6047) (width 1) (layer "B.Cu") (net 5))
 (segment (start 183.3328 125.0678) (end 179.5519 125.0678) (width 1) (layer "B.Cu") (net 5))
 (segment (start 242.8 129.235) (end 239.9889 126.4239) (width 1) (layer "B.Cu") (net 5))
 (segment (start 239.9889 126.4239) (end 236.3111 126.4239) (width 1) (layer "B.Cu") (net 5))
 (segment (start 189.1074 127.6276) (end 195.0926 127.6276) (width 1) (layer "B.Cu") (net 5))
 (segment (start 195.0926 127.6276) (end 196.7 129.235) (width 1) (layer "B.Cu") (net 5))
 (segment (start 169.1 129.235) (end 170.7303 127.6047) (width 1) (layer "B.Cu") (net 5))
 (segment (start 179.5519 125.0678) (end 178.3 126.3197) (width 1) (layer "B.Cu") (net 5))
 (segment (start 178.3 127.6047) (end 178.3 129.235) (width 1) (layer "B.Cu") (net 5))
 (segment (start 236.3111 126.4239) (end 233.5 129.235) (width 1) (layer "B.Cu") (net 5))
 (segment (start 225.9029 127.6321) (end 231.8971 127.6321) (width 1) (layer "B.Cu") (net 5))
 (segment (start 187.5 129.235) (end 183.3328 125.0678) (width 1) (layer "B.Cu") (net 5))
 (segment (start 224.3 129.235) (end 225.9029 127.6321) (width 1) (layer "B.Cu") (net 5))
 (segment (start 231.8971 127.6321) (end 233.5 129.235) (width 1) (layer "B.Cu") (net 5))
 (segment (start 186.1006 133.3753) (end 184.5003 131.775) (width 1) (layer "F.Cu") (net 1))
 (segment (start 188.8994 133.3753) (end 186.1006 133.3753) (width 1) (layer "F.Cu") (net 1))
 (segment (start 190.4997 131.775) (end 188.8994 133.3753) (width 1) (layer "F.Cu") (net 1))
 (segment (start 192.1 131.775) (end 190.4997 131.775) (width 1) (layer "F.Cu") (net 1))
 (segment (start 182.9 131.775) (end 184.5003 131.775) (width 1) (layer "F.Cu") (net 1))
 (segment (start 182.6025 134.5367) (end 181.4211 135.7181) (width 1) (layer "B.Cu") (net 1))
 (segment (start 201.3 134) (end 201.3 133.3754) (width 1) (layer "B.Cu") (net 1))
 (segment (start 192.1 131.775) (end 193.7003 131.775) (width 1) (layer "B.Cu") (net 1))
 (segment (start 195.3007 133.3754) (end 201.3 133.3754) (width 1) (layer "B.Cu") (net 1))
 (segment (start 201.3 133.3754) (end 201.3 131.775) (width 1) (layer "B.Cu") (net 1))
 (segment (start 180.65 131.65) (end 182.3253 131.65) (width 1) (layer "B.Cu") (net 1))
 (segment (start 202.7 135.4) (end 201.3 134) (width 1) (layer "B.Cu") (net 1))
 (segment (start 182.9 131.775) (end 182.7478 131.9272) (width 1) (layer "B.Cu") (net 1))
 (segment (start 181.4211 135.7181) (end 177.6431 135.7181) (width 1) (layer "B.Cu") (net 1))
 (segment (start 177.6431 135.7181) (end 173.7 131.775) (width 1) (layer "B.Cu") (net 1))
 (segment (start 193.7003 131.775) (end 195.3007 133.3754) (width 1) (layer "B.Cu") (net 1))
 (segment (start 182.7478 131.9272) (end 182.6025 131.9272) (width 1) (layer "B.Cu") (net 1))
 (segment (start 182.6025 131.9272) (end 182.3253 131.65) (width 1) (layer "B.Cu") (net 1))
 (segment (start 182.6025 131.9272) (end 182.6025 134.5367) (width 1) (layer "B.Cu") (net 1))
 (segment (start 191.4747 135.4) (end 195.0997 131.775) (width 1) (layer "F.Cu") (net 2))
 (segment (start 205.9 131.775) (end 207.5003 131.775) (width 1) (layer "F.Cu") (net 2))
 (segment (start 185.5597 135.4) (end 185.2593 135.7004) (width 1) (layer "F.Cu") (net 2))
 (segment (start 178.3 134.1293) (end 178.3 133.3754) (width 1) (layer "F.Cu") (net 2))
 (segment (start 170.7003 131.775) (end 172.3007 133.3754) (width 1) (layer "F.Cu") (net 2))
 (segment (start 187.46 135.4) (end 185.5597 135.4) (width 1) (layer "F.Cu") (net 2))
 (segment (start 230.2994 133.3753) (end 227.5006 133.3753) (width 1) (layer "F.Cu") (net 2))
 (segment (start 224.3 131.775) (end 225.6002 131.775) (width 1) (layer "F.Cu") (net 2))
 (segment (start 178.3 133.3754) (end 178.3 131.775) (width 1) (layer "F.Cu") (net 2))
 (segment (start 225.9003 128.5324) (end 223.7428 126.3749) (width 1) (layer "F.Cu") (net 2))
 (segment (start 185.2593 135.7004) (end 179.8711 135.7004) (width 1) (layer "F.Cu") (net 2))
 (segment (start 179.8711 135.7004) (end 178.3 134.1293) (width 1) (layer "F.Cu") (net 2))
 (segment (start 207.5003 131.775) (end 209.1006 133.3753) (width 1) (layer "F.Cu") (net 2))
 (segment (start 169.1 131.775) (end 170.7003 131.775) (width 1) (layer "F.Cu") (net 2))
 (segment (start 215.1 131.775) (end 213.4997 131.775) (width 1) (layer "F.Cu") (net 2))
 (segment (start 215.6901 126.3749) (end 213.4997 128.5653) (width 1) (layer "F.Cu") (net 2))
 (segment (start 231.8997 131.775) (end 230.2994 133.3753) (width 1) (layer "F.Cu") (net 2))
 (segment (start 209.1006 133.3753) (end 211.8994 133.3753) (width 1) (layer "F.Cu") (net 2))
 (segment (start 211.8994 133.3753) (end 213.4997 131.775) (width 1) (layer "F.Cu") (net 2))
 (segment (start 172.3007 133.3754) (end 178.3 133.3754) (width 1) (layer "F.Cu") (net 2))
 (segment (start 227.5006 133.3753) (end 225.9003 131.775) (width 1) (layer "F.Cu") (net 2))
 (segment (start 225.9003 131.775) (end 225.9003 128.5324) (width 1) (layer "F.Cu") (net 2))
 (segment (start 196.7 131.775) (end 195.0997 131.775) (width 1) (layer "F.Cu") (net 2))
 (segment (start 223.7428 126.3749) (end 215.6901 126.3749) (width 1) (layer "F.Cu") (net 2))
 (segment (start 233.5 131.775) (end 231.8997 131.775) (width 1) (layer "F.Cu") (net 2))
 (segment (start 225.6002 131.775) (end 225.9003 131.775) (width 1) (layer "F.Cu") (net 2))
 (segment (start 187.46 135.4) (end 191.4747 135.4) (width 1) (layer "F.Cu") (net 2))
 (segment (start 213.4997 128.5653) (end 213.4997 131.775) (width 1) (layer "F.Cu") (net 2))
 (segment (start 182.5784 126.65) (end 180.65 126.65) (width 1) (layer "B.Cu") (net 2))
 (segment (start 242.8 131.5575) (end 242.8 131.775) (width 1) (layer "B.Cu") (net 2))
 (segment (start 187.5 131.5716) (end 182.5784 126.65) (width 1) (layer "B.Cu") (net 2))
 (segment (start 187.5 131.775) (end 187.5 131.5716) (width 1) (layer "B.Cu") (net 2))
 (segment (start 238.8719 127.6294) (end 242.8 131.5575) (width 1) (layer "B.Cu") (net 2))
 (segment (start 200.8397 127.3936) (end 201.7532 127.3936) (width 1) (layer "B.Cu") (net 2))
 (segment (start 196.7 131.775) (end 196.7 131.5333) (width 1) (layer "B.Cu") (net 2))
 (segment (start 187.46 133.4997) (end 187.5 133.4597) (width 1) (layer "B.Cu") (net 2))
 (segment (start 200.8397 127.3936) (end 200.8397 125.6) (width 1) (layer "B.Cu") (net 2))
 (segment (start 202.74 125.6) (end 200.8397 125.6) (width 1) (layer "B.Cu") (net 2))
 (segment (start 233.5 131.775) (end 233.5 131.5644) (width 1) (layer "B.Cu") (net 2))
 (segment (start 187.46 135.4) (end 187.46 133.4997) (width 1) (layer "B.Cu") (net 2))
 (segment (start 201.7532 127.3936) (end 205.9 131.5404) (width 1) (layer "B.Cu") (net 2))
 (segment (start 187.5 133.4597) (end 187.5 131.775) (width 1) (layer "B.Cu") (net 2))
 (segment (start 196.7 131.5333) (end 200.8397 127.3936) (width 1) (layer "B.Cu") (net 2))
 (segment (start 205.9 131.5404) (end 205.9 131.775) (width 1) (layer "B.Cu") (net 2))
 (segment (start 237.435 127.6294) (end 238.8719 127.6294) (width 1) (layer "B.Cu") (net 2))
 (segment (start 233.5 131.5644) (end 237.435 127.6294) (width 1) (layer "B.Cu") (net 2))
 (segment (start 199.9284 125.6) (end 201.8287 127.5003) (width 1) (layer "F.Cu") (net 3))
 (segment (start 178.9626 125.6506) (end 179.5178 125.0954) (width 1) (layer "F.Cu") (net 3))
 (segment (start 179.5178 125.0954) (end 186.9954 125.0954) (width 1) (layer "F.Cu") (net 3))
 (segment (start 187.5 125.6) (end 199.9284 125.6) (width 1) (layer "F.Cu") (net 3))
 (segment (start 233.6766 134.6381) (end 236.5397 131.775) (width 1) (layer "F.Cu") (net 3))
 (segment (start 224.1634 134.6381) (end 233.6766 134.6381) (width 1) (layer "F.Cu") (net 3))
 (segment (start 201.8287 127.5003) (end 206.4503 127.5003) (width 1) (layer "F.Cu") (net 3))
 (segment (start 206.4503 127.5003) (end 210.5 131.55) (width 1) (layer "F.Cu") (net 3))
 (segment (start 221.3003 131.775) (end 224.1634 134.6381) (width 1) (layer "F.Cu") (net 3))
 (segment (start 210.5 131.55) (end 210.5 131.775) (width 1) (layer "F.Cu") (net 3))
 (segment (start 238.14 131.775) (end 236.5397 131.775) (width 1) (layer "F.Cu") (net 3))
 (segment (start 219.7 131.775) (end 221.3003 131.775) (width 1) (layer "F.Cu") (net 3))
 (segment (start 186.9954 125.0954) (end 187.5 125.6) (width 1) (layer "F.Cu") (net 3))
 (segment (start 178.9626 127.6336) (end 178.9626 125.6506) (width 1) (layer "F.Cu") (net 3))
 (segment (start 180.479 129.15) (end 178.9626 127.6336) (width 1) (layer "F.Cu") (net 3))
 (segment (start 180.65 129.15) (end 180.479 129.15) (width 1) (layer "F.Cu") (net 3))
 (segment (start 228.9 131.775) (end 230.5003 131.775) (width 1) (layer "B.Cu") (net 3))
 (segment (start 238.14 131.775) (end 236.5397 131.775) (width 1) (layer "B.Cu") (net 3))
 (segment (start 219.7 131.775) (end 218.0997 131.775) (width 1) (layer "B.Cu") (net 3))
 (segment (start 234.9394 133.3753) (end 232.1006 133.3753) (width 1) (layer "B.Cu") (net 3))
 (segment (start 210.5 131.775) (end 212.1003 131.775) (width 1) (layer "B.Cu") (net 3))
 (segment (start 212.1003 131.775) (end 213.7006 133.3753) (width 1) (layer "B.Cu") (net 3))
 (segment (start 216.4994 133.3753) (end 218.0997 131.775) (width 1) (layer "B.Cu") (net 3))
 (segment (start 236.5397 131.775) (end 234.9394 133.3753) (width 1) (layer "B.Cu") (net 3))
 (segment (start 213.7006 133.3753) (end 216.4994 133.3753) (width 1) (layer "B.Cu") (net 3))
 (segment (start 232.1006 133.3753) (end 230.5003 131.775) (width 1) (layer "B.Cu") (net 3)))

